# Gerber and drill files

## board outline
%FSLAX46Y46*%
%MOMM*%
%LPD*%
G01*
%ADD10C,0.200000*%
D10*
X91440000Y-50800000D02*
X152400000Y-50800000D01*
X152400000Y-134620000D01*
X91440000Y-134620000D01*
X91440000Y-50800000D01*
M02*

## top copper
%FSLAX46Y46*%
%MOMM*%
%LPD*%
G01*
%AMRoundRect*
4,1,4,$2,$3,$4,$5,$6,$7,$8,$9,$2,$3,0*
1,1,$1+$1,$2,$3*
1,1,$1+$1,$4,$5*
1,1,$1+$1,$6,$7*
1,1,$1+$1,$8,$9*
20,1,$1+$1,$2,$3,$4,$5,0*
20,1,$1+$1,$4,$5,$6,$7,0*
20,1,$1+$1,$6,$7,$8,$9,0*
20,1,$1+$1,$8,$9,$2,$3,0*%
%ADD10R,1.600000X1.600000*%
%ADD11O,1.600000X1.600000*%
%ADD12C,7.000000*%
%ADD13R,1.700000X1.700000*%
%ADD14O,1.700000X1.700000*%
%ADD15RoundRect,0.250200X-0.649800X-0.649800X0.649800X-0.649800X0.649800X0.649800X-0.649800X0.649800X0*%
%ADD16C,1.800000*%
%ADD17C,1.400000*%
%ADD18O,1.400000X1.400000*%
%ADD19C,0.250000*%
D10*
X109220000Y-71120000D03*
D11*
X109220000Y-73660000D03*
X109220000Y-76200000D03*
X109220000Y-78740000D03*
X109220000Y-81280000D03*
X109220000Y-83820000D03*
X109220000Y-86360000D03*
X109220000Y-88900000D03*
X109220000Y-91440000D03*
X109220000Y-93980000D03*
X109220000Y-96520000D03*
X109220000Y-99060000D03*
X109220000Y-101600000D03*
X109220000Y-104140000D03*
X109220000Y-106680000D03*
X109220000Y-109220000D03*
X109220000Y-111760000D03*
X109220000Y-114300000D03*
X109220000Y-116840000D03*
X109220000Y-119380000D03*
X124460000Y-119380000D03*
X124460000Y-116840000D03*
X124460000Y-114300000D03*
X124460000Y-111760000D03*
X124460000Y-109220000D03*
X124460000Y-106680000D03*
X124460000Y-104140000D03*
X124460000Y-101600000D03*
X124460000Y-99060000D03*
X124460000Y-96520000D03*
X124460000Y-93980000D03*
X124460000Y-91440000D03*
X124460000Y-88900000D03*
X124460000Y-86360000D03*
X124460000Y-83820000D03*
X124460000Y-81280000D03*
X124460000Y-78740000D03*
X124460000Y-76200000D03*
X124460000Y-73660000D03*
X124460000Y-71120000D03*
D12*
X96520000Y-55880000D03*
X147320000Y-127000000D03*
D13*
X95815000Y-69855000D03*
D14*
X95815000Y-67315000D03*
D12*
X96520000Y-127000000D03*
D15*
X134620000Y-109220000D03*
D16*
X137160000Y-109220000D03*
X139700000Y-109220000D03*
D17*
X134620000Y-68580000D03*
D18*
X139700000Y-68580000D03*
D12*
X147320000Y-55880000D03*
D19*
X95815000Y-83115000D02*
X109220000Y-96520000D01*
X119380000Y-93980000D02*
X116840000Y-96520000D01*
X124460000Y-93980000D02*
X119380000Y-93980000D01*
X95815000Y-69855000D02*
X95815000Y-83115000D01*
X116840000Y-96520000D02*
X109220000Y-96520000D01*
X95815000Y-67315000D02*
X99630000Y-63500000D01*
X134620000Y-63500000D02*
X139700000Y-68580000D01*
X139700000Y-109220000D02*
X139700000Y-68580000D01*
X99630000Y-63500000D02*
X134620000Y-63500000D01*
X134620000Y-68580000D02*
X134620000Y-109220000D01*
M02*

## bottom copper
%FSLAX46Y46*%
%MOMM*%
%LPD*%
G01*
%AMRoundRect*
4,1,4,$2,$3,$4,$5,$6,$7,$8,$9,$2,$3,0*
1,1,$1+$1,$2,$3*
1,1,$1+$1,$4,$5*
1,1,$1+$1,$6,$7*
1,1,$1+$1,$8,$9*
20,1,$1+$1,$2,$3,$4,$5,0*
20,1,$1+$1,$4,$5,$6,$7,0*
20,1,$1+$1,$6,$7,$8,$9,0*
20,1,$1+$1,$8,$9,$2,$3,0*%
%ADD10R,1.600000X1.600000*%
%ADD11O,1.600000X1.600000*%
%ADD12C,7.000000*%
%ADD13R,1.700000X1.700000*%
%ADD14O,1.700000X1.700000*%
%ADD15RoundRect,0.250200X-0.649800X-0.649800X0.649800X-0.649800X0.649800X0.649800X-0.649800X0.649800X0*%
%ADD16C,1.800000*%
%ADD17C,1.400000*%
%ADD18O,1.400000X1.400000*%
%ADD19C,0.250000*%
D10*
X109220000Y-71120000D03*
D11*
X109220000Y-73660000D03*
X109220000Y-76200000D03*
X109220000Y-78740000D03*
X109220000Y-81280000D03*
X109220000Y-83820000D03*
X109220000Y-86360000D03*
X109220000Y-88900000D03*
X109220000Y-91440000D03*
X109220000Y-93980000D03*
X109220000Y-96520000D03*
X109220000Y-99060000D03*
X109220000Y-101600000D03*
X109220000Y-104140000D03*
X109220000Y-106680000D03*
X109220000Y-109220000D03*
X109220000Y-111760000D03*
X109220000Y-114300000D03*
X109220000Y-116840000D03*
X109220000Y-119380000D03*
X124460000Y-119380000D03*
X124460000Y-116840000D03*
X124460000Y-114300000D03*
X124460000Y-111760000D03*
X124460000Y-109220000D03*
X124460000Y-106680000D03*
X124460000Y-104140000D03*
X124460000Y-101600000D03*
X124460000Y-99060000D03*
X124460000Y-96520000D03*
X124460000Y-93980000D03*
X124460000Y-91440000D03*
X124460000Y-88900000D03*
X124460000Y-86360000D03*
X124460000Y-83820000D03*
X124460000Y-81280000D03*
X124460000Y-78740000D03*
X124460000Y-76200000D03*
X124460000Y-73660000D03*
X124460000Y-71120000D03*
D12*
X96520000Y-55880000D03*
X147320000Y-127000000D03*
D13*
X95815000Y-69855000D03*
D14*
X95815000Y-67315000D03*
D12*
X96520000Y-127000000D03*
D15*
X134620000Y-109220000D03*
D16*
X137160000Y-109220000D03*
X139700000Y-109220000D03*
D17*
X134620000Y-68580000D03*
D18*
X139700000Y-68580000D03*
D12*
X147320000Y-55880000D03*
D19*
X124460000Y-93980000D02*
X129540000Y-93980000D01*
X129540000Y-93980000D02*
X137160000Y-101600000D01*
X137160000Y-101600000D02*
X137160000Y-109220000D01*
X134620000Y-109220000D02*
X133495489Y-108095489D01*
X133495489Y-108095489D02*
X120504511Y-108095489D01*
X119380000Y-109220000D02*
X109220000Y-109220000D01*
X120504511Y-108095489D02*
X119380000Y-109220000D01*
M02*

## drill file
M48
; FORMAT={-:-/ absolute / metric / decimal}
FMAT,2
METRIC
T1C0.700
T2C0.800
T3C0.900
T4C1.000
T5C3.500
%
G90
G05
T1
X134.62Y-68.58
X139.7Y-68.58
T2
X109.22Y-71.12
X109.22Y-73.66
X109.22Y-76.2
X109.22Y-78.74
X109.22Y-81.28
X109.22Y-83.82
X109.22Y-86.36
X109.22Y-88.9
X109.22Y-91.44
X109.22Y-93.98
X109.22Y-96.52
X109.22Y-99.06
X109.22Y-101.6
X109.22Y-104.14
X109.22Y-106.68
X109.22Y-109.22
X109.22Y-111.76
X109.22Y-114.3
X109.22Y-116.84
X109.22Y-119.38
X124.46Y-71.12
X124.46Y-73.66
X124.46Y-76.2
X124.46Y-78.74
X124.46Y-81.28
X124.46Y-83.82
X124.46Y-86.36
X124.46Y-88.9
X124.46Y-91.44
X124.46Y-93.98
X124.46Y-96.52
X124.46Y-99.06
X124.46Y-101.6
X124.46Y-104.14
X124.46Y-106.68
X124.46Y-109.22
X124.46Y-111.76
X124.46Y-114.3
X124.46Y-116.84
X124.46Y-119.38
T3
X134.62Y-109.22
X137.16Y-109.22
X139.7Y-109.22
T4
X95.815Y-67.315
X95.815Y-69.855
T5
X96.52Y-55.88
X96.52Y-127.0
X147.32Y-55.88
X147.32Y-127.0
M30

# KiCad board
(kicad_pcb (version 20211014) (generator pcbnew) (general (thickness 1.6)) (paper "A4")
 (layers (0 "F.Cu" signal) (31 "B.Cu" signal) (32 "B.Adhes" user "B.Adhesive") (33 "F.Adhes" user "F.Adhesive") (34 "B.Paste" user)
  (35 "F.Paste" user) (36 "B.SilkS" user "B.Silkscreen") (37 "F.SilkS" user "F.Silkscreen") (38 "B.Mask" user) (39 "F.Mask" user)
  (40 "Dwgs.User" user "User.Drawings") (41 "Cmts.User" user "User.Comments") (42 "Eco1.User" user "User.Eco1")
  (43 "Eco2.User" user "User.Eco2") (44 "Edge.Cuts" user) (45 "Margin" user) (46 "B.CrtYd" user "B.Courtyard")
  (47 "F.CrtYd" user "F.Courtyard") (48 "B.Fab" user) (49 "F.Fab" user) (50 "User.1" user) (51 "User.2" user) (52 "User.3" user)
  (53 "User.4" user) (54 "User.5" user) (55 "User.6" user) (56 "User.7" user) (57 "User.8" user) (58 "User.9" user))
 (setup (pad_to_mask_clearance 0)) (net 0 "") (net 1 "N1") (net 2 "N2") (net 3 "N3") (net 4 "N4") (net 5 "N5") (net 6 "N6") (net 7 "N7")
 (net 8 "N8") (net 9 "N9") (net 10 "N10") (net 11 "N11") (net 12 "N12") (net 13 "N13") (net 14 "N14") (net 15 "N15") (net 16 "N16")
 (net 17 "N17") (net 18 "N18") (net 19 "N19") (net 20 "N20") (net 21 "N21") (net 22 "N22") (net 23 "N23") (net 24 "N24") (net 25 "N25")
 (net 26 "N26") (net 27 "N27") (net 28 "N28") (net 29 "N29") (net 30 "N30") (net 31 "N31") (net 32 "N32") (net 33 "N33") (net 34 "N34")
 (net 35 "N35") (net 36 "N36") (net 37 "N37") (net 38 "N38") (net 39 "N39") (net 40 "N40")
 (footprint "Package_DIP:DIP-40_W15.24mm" (layer "F.Cu") (at 109.22 71.12)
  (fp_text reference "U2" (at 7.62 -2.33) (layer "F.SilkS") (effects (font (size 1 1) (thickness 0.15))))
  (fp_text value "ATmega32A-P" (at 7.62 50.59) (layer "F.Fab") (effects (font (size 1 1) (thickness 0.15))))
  (pad "1" thru_hole rect (at 0 0) (size 1.6 1.6) (drill 0.8) (layers *.Cu *.Mask) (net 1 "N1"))
  (pad "2" thru_hole oval (at 0 2.54) (size 1.6 1.6) (drill 0.8) (layers *.Cu *.Mask) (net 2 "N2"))
  (pad "3" thru_hole oval (at 0 5.08) (size 1.6 1.6) (drill 0.8) (layers *.Cu *.Mask) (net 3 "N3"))
  (pad "4" thru_hole oval (at 0 7.62) (size 1.6 1.6) (drill 0.8) (layers *.Cu *.Mask) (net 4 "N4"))
  (pad "5" thru_hole oval (at 0 10.16) (size 1.6 1.6) (drill 0.8) (layers *.Cu *.Mask) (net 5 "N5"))
  (pad "6" thru_hole oval (at 0 12.7) (size 1.6 1.6) (drill 0.8) (layers *.Cu *.Mask) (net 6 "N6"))
  (pad "7" thru_hole oval (at 0 15.24) (size 1.6 1.6) (drill 0.8) (layers *.Cu *.Mask) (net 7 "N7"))
  (pad "8" thru_hole oval (at 0 17.78) (size 1.6 1.6) (drill 0.8) (layers *.Cu *.Mask) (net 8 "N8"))
  (pad "9" thru_hole oval (at 0 20.32) (size 1.6 1.6) (drill 0.8) (layers *.Cu *.Mask) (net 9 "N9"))
  (pad "10" thru_hole oval (at 0 22.86) (size 1.6 1.6) (drill 0.8) (layers *.Cu *.Mask) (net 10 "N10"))
  (pad "11" thru_hole oval (at 0 25.4) (size 1.6 1.6) (drill 0.8) (layers *.Cu *.Mask) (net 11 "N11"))
  (pad "12" thru_hole oval (at 0 27.94) (size 1.6 1.6) (drill 0.8) (layers *.Cu *.Mask) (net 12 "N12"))
  (pad "13" thru_hole oval (at 0 30.48) (size 1.6 1.6) (drill 0.8) (layers *.Cu *.Mask) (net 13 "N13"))
  (pad "14" thru_hole oval (at 0 33.02) (size 1.6 1.6) (drill 0.8) (layers *.Cu *.Mask) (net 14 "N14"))
  (pad "15" thru_hole oval (at 0 35.56) (size 1.6 1.6) (drill 0.8) (layers *.Cu *.Mask) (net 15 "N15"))
  (pad "16" thru_hole oval (at 0 38.1) (size 1.6 1.6) (drill 0.8) (layers *.Cu *.Mask) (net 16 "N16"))
  (pad "17" thru_hole oval (at 0 40.64) (size 1.6 1.6) (drill 0.8) (layers *.Cu *.Mask) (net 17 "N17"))
  (pad "18" thru_hole oval (at 0 43.18) (size 1.6 1.6) (drill 0.8) (layers *.Cu *.Mask) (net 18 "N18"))
  (pad "19" thru_hole oval (at 0 45.72) (size 1.6 1.6) (drill 0.8) (layers *.Cu *.Mask) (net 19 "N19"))
  (pad "20" thru_hole oval (at 0 48.26) (size 1.6 1.6) (drill 0.8) (layers *.Cu *.Mask) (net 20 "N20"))
  (pad "21" thru_hole oval (at 15.24 48.26) (size 1.6 1.6) (drill 0.8) (layers *.Cu *.Mask) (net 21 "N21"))
  (pad "22" thru_hole oval (at 15.24 45.72) (size 1.6 1.6) (drill 0.8) (layers *.Cu *.Mask) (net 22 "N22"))
  (pad "23" thru_hole oval (at 15.24 43.18) (size 1.6 1.6) (drill 0.8) (layers *.Cu *.Mask) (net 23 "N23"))
  (pad "24" thru_hole oval (at 15.24 40.64) (size 1.6 1.6) (drill 0.8) (layers *.Cu *.Mask) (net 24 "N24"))
  (pad "25" thru_hole oval (at 15.24 38.1) (size 1.6 1.6) (drill 0.8) (layers *.Cu *.Mask) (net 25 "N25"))
  (pad "26" thru_hole oval (at 15.24 35.56) (size 1.6 1.6) (drill 0.8) (layers *.Cu *.Mask) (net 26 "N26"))
  (pad "27" thru_hole oval (at 15.24 33.02) (size 1.6 1.6) (drill 0.8) (layers *.Cu *.Mask) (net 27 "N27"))
  (pad "28" thru_hole oval (at 15.24 30.48) (size 1.6 1.6) (drill 0.8) (layers *.Cu *.Mask) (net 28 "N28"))
  (pad "29" thru_hole oval (at 15.24 27.94) (size 1.6 1.6) (drill 0.8) (layers *.Cu *.Mask) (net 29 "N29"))
  (pad "30" thru_hole oval (at 15.24 25.4) (size 1.6 1.6) (drill 0.8) (layers *.Cu *.Mask) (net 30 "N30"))
  (pad "31" thru_hole oval (at 15.24 22.86) (size 1.6 1.6) (drill 0.8) (layers *.Cu *.Mask) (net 11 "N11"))
  (pad "32" thru_hole oval (at 15.24 20.32) (size 1.6 1.6) (drill 0.8) (layers *.Cu *.Mask) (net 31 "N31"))
  (pad "33" thru_hole oval (at 15.24 17.78) (size 1.6 1.6) (drill 0.8) (layers *.Cu *.Mask) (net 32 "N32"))
  (pad "34" thru_hole oval (at 15.24 15.24) (size 1.6 1.6) (drill 0.8) (layers *.Cu *.Mask) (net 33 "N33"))
  (pad "35" thru_hole oval (at 15.24 12.7) (size 1.6 1.6) (drill 0.8) (layers *.Cu *.Mask) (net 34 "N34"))
  (pad "36" thru_hole oval (at 15.24 10.16) (size 1.6 1.6) (drill 0.8) (layers *.Cu *.Mask) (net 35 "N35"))
  (pad "37" thru_hole oval (at 15.24 7.62) (size 1.6 1.6) (drill 0.8) (layers *.Cu *.Mask) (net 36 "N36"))
  (pad "38" thru_hole oval (at 15.24 5.08) (size 1.6 1.6) (drill 0.8) (layers *.Cu *.Mask) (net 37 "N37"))
  (pad "39" thru_hole oval (at 15.24 2.54) (size 1.6 1.6) (drill 0.8) (layers *.Cu *.Mask) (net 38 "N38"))
  (pad "40" thru_hole oval (at 15.24 0) (size 1.6 1.6) (drill 0.8) (layers *.Cu *.Mask) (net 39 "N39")))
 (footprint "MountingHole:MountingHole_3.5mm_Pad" (layer "F.Cu") (at 96.52 55.88)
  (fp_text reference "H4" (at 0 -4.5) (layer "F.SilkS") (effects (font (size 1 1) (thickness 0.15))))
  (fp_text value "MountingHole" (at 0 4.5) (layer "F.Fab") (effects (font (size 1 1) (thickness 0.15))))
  (pad "1" thru_hole circle (at 0 0) (size 7 7) (drill 3.5) (layers *.Cu *.Mask)))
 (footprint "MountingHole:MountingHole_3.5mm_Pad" (layer "F.Cu") (at 147.32 127)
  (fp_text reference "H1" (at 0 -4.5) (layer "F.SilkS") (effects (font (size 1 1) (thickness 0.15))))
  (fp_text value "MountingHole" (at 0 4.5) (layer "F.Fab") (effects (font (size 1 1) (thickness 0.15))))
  (pad "1" thru_hole circle (at 0 0) (size 7 7) (drill 3.5) (layers *.Cu *.Mask)))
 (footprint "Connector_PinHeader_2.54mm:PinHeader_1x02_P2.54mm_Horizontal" (layer "F.Cu") (at 95.815 69.855 180)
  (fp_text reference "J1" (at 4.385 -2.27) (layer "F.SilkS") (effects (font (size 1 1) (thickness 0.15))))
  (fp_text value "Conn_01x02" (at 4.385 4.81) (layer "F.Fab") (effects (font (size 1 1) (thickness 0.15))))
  (pad "1" thru_hole rect (at 0 0 180) (size 1.7 1.7) (drill 1) (layers *.Cu *.Mask) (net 11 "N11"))
  (pad "2" thru_hole oval (at 0 2.54 180) (size 1.7 1.7) (drill 1) (layers *.Cu *.Mask) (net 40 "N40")))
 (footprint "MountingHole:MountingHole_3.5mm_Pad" (layer "F.Cu") (at 96.52 127)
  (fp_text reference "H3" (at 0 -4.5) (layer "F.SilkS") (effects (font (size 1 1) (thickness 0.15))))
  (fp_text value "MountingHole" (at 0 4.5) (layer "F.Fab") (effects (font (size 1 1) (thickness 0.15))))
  (pad "1" thru_hole circle (at 0 0) (size 7 7) (drill 3.5) (layers *.Cu *.Mask)))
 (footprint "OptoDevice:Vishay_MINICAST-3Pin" (layer "F.Cu") (at 134.62 109.22)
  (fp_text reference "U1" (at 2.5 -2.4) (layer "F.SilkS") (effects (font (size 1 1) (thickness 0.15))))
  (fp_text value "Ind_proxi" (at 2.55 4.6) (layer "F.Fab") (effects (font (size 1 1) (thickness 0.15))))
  (pad "1" thru_hole roundrect (at 0 0) (size 1.8 1.8) (drill 0.9) (layers *.Cu *.Mask) (roundrect_rratio 0.139) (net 16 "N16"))
  (pad "2" thru_hole circle (at 2.54 0) (size 1.8 1.8) (drill 0.9) (layers *.Cu *.Mask) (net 11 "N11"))
  (pad "3" thru_hole circle (at 5.08 0) (size 1.8 1.8) (drill 0.9) (layers *.Cu *.Mask) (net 40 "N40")))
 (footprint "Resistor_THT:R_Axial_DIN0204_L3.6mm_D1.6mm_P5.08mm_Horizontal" (layer "F.Cu") (at 134.62 68.58)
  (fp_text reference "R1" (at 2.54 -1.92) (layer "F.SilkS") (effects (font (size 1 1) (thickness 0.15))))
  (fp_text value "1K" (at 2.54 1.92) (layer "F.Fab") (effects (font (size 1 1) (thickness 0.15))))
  (pad "1" thru_hole circle (at 0 0) (size 1.4 1.4) (drill 0.7) (layers *.Cu *.Mask) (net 16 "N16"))
  (pad "2" thru_hole oval (at 5.08 0) (size 1.4 1.4) (drill 0.7) (layers *.Cu *.Mask) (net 40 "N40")))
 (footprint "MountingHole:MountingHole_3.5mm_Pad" (layer "F.Cu") (at 147.32 55.88)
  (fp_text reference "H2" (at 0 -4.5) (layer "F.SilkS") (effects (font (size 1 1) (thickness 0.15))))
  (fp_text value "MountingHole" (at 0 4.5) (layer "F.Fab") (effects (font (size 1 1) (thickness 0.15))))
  (pad "1" thru_hole circle (at 0 0) (size 7 7) (drill 3.5) (layers *.Cu *.Mask)))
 (gr_rect (start 91.44 50.8) (end 152.4 134.62) (layer "Edge.Cuts") (width 0.2) (fill none))
 (segment (start 95.815 83.115) (end 109.22 96.52) (width 0.25) (layer "F.Cu") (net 11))
 (segment (start 119.38 93.98) (end 116.84 96.52) (width 0.25) (layer "F.Cu") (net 11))
 (segment (start 124.46 93.98) (end 119.38 93.98) (width 0.25) (layer "F.Cu") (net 11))
 (segment (start 95.815 69.855) (end 95.815 83.115) (width 0.25) (layer "F.Cu") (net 11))
 (segment (start 116.84 96.52) (end 109.22 96.52) (width 0.25) (layer "F.Cu") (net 11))
 (segment (start 124.46 93.98) (end 129.54 93.98) (width 0.25) (layer "B.Cu") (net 11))
 (segment (start 129.54 93.98) (end 137.16 101.6) (width 0.25) (layer "B.Cu") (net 11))
 (segment (start 137.16 101.6) (end 137.16 109.22) (width 0.25) (layer "B.Cu") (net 11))
 (segment (start 95.815 67.315) (end 99.63 63.5) (width 0.25) (layer "F.Cu") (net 40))
 (segment (start 134.62 63.5) (end 139.7 68.58) (width 0.25) (layer "F.Cu") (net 40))
 (segment (start 139.7 109.22) (end 139.7 68.58) (width 0.25) (layer "F.Cu") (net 40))
 (segment (start 99.63 63.5) (end 134.62 63.5) (width 0.25) (layer "F.Cu") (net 40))
 (segment (start 134.62 68.58) (end 134.62 109.22) (width 0.25) (layer "F.Cu") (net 16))
 (segment (start 134.62 109.22) (end 133.495489 108.095489) (width 0.25) (layer "B.Cu") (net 16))
 (segment (start 133.495489 108.095489) (end 120.504511 108.095489) (width 0.25) (layer "B.Cu") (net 16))
 (segment (start 119.38 109.22) (end 109.22 109.22) (width 0.25) (layer "B.Cu") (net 16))
 (segment (start 120.504511 108.095489) (end 119.38 109.22) (width 0.25) (layer "B.Cu") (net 16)))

